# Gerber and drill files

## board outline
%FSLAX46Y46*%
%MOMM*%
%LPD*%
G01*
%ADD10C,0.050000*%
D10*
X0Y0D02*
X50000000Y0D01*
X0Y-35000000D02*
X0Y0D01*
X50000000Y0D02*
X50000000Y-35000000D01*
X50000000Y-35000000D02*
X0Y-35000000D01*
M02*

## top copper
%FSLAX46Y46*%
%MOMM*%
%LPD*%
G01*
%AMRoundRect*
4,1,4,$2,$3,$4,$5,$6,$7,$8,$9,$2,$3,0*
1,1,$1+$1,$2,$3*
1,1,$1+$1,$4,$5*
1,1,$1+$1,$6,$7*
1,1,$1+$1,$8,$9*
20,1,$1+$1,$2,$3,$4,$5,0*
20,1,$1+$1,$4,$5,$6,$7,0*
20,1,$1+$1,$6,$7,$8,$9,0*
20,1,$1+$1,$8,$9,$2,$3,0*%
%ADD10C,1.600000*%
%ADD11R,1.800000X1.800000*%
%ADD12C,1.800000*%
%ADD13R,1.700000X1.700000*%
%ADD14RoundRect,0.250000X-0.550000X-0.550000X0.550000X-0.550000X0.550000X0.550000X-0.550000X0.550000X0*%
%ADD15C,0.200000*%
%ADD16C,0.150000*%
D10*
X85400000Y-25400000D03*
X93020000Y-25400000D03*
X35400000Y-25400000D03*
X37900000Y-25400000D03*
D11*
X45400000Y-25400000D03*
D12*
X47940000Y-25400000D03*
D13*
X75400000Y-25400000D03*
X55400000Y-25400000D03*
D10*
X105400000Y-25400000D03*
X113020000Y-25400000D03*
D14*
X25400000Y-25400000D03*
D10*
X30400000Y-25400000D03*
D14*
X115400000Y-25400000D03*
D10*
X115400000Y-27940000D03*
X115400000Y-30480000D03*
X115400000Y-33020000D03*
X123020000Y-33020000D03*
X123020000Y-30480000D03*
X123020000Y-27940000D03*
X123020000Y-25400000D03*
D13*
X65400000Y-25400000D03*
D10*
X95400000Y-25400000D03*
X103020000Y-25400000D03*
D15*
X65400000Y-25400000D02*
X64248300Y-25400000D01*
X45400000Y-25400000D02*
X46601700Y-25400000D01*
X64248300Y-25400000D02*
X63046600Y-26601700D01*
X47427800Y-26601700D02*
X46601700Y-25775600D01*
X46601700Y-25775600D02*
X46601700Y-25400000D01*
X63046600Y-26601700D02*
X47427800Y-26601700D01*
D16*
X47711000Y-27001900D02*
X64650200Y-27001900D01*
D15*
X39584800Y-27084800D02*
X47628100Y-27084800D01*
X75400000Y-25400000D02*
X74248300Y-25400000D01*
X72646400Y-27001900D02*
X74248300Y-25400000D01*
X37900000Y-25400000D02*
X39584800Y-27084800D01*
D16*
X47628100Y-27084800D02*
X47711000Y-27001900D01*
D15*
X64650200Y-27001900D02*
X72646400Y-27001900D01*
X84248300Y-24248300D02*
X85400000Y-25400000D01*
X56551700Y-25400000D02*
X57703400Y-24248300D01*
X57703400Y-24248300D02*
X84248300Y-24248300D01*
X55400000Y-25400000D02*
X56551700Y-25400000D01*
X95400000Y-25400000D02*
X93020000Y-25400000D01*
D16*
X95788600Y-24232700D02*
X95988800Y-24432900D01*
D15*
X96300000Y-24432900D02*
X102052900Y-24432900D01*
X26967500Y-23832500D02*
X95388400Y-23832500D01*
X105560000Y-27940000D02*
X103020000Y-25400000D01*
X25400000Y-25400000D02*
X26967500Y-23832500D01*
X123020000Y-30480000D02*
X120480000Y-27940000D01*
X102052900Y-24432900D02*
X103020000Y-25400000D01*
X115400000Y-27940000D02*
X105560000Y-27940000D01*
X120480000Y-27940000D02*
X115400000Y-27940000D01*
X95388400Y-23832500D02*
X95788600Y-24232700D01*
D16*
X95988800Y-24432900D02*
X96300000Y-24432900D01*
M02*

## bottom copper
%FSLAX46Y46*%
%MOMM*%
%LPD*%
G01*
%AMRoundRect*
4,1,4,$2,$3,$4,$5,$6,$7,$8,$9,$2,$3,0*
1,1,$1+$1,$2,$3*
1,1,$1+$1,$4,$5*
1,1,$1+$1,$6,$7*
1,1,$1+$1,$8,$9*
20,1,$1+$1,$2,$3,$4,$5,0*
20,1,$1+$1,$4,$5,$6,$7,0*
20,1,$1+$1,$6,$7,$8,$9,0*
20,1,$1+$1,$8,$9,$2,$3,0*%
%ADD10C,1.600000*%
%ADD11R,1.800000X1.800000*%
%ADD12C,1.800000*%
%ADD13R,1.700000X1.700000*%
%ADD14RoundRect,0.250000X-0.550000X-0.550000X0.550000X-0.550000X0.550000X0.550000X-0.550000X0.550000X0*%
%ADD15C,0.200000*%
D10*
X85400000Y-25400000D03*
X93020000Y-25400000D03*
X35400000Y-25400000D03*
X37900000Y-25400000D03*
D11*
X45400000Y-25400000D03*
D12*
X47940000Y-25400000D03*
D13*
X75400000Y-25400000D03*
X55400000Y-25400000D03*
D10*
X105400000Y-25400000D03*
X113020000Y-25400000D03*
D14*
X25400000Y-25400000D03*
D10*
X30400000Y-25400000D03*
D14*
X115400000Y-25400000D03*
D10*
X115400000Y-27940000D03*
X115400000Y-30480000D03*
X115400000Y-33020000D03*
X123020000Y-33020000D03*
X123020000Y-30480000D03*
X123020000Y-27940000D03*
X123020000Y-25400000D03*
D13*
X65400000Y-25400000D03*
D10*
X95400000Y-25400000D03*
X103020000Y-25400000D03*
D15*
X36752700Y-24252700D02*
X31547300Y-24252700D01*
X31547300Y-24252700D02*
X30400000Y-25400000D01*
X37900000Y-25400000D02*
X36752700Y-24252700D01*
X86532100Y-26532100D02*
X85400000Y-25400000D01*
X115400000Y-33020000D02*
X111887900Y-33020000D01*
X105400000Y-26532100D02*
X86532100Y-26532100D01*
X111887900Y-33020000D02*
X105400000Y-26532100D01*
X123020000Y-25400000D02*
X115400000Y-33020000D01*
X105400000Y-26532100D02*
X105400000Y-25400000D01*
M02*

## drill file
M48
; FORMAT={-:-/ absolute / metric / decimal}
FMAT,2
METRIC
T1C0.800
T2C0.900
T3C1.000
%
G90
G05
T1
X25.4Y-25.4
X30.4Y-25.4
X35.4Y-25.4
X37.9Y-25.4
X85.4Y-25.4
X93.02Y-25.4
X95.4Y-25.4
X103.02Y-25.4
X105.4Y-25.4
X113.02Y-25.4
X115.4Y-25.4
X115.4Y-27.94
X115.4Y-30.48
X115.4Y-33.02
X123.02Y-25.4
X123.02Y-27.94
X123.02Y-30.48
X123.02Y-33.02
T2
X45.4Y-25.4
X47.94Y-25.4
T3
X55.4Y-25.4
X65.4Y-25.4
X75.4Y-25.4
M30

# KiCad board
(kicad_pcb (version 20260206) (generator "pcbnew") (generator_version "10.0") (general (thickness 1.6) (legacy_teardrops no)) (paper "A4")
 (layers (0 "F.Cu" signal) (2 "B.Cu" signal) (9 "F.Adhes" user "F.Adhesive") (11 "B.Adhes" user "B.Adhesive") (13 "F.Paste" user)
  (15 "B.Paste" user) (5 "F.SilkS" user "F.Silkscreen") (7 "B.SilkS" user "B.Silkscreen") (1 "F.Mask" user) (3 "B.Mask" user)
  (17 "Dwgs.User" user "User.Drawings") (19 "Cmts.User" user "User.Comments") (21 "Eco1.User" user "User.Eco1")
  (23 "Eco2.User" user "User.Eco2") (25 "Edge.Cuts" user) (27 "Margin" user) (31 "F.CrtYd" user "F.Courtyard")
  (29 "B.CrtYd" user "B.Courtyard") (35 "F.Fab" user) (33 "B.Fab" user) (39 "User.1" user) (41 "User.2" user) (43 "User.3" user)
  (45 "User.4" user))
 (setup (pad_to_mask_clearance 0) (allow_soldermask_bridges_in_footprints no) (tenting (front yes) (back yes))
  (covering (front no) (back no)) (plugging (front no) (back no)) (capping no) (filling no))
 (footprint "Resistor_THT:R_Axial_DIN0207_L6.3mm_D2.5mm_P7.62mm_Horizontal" (layer "F.Cu") (at 85.4 25.4)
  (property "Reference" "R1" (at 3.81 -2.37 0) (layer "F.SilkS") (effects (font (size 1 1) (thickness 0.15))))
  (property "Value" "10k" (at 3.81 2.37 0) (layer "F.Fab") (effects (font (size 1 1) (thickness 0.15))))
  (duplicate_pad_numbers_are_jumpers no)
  (pad "1" thru_hole circle (at 0 0) (size 1.6 1.6) (drill 0.8) (layers "*.Cu" "*.Mask") (remove_unused_layers no) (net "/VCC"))
  (pad "2" thru_hole circle (at 7.62 0) (size 1.6 1.6) (drill 0.8) (layers "*.Cu" "*.Mask") (remove_unused_layers no) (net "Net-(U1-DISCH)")))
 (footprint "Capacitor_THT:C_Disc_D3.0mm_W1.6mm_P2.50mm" (layer "F.Cu") (at 35.4 25.4)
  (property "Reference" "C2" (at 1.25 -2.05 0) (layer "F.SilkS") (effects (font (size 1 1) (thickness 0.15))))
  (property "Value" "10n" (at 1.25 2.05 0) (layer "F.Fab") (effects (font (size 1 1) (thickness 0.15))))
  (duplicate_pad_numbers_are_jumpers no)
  (pad "1" thru_hole circle (at 0 0) (size 1.6 1.6) (drill 0.8) (layers "*.Cu" "*.Mask") (remove_unused_layers no) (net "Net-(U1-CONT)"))
  (pad "2" thru_hole circle (at 2.5 0) (size 1.6 1.6) (drill 0.8) (layers "*.Cu" "*.Mask") (remove_unused_layers no) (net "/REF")))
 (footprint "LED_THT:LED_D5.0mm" (layer "F.Cu") (at 45.4 25.4)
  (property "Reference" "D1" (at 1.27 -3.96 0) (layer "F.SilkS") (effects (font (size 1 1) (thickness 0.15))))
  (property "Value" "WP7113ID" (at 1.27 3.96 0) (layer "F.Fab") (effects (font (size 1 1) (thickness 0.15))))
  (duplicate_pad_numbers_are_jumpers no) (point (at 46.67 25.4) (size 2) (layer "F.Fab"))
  (pad "1" thru_hole rect (at 0 0) (size 1.8 1.8) (drill 0.9) (layers "*.Cu" "*.Mask") (remove_unused_layers no) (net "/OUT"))
  (pad "2" thru_hole circle (at 2.54 0) (size 1.8 1.8) (drill 0.9) (layers "*.Cu" "*.Mask") (remove_unused_layers no) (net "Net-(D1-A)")))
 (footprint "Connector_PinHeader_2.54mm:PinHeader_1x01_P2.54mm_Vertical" (layer "F.Cu") (at 75.4 25.4)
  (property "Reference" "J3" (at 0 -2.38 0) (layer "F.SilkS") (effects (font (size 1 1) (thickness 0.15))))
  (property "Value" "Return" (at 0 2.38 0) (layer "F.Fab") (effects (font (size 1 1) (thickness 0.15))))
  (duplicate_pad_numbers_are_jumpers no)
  (pad "1" thru_hole rect (at 0 0) (size 1.7 1.7) (drill 1) (layers "*.Cu" "*.Mask") (remove_unused_layers no) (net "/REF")))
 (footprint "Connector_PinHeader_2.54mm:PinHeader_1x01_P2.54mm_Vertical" (layer "F.Cu") (at 55.4 25.4)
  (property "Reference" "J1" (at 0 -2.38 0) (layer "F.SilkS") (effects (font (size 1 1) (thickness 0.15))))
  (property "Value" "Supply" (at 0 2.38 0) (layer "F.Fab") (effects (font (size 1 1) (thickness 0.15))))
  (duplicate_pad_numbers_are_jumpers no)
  (pad "1" thru_hole rect (at 0 0) (size 1.7 1.7) (drill 1) (layers "*.Cu" "*.Mask") (remove_unused_layers no) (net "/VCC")))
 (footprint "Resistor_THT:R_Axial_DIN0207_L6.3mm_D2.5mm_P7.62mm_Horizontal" (layer "F.Cu") (at 105.4 25.4)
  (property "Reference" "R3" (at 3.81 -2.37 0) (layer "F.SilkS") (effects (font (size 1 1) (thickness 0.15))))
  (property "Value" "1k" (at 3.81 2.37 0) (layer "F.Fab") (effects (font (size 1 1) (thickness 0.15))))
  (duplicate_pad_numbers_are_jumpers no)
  (pad "1" thru_hole circle (at 0 0) (size 1.6 1.6) (drill 0.8) (layers "*.Cu" "*.Mask") (remove_unused_layers no) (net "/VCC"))
  (pad "2" thru_hole circle (at 7.62 0) (size 1.6 1.6) (drill 0.8) (layers "*.Cu" "*.Mask") (remove_unused_layers no) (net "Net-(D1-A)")))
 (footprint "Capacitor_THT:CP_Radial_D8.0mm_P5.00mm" (layer "F.Cu") (at 25.4 25.4)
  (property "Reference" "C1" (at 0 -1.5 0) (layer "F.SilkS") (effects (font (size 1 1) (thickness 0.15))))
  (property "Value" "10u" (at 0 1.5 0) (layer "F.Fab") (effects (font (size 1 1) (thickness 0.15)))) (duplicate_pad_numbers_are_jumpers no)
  (pad "1" thru_hole roundrect (at 0 0) (size 1.6 1.6) (drill 0.8) (layers "*.Cu" "*.Mask") (remove_unused_layers no)
   (roundrect_rratio 0.15625) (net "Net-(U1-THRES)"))
  (pad "2" thru_hole circle (at 5 0) (size 1.6 1.6) (drill 0.8) (layers "*.Cu" "*.Mask") (remove_unused_layers no) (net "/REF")))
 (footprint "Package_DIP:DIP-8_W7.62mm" (layer "F.Cu") (at 115.4 25.4)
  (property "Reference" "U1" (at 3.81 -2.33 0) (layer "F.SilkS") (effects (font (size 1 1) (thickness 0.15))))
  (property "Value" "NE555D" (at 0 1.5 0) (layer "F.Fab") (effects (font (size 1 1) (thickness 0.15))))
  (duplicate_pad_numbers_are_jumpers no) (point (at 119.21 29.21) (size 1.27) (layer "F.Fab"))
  (pad "1" thru_hole roundrect (at 0 0) (size 1.6 1.6) (drill 0.8) (layers "*.Cu" "*.Mask") (remove_unused_layers no)
   (roundrect_rratio 0.15625) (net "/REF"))
  (pad "2" thru_hole circle (at 0 2.54) (size 1.6 1.6) (drill 0.8) (layers "*.Cu" "*.Mask") (remove_unused_layers no) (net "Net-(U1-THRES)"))
  (pad "3" thru_hole circle (at 0 5.08) (size 1.6 1.6) (drill 0.8) (layers "*.Cu" "*.Mask") (remove_unused_layers no) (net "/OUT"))
  (pad "4" thru_hole circle (at 0 7.62) (size 1.6 1.6) (drill 0.8) (layers "*.Cu" "*.Mask") (remove_unused_layers no) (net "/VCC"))
  (pad "5" thru_hole circle (at 7.62 7.62) (size 1.6 1.6) (drill 0.8) (layers "*.Cu" "*.Mask") (remove_unused_layers no)
   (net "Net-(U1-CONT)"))
  (pad "6" thru_hole circle (at 7.62 5.08) (size 1.6 1.6) (drill 0.8) (layers "*.Cu" "*.Mask") (remove_unused_layers no)
   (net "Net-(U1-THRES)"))
  (pad "7" thru_hole circle (at 7.62 2.54) (size 1.6 1.6) (drill 0.8) (layers "*.Cu" "*.Mask") (remove_unused_layers no)
   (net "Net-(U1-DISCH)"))
  (pad "8" thru_hole circle (at 7.62 0) (size 1.6 1.6) (drill 0.8) (layers "*.Cu" "*.Mask") (remove_unused_layers no) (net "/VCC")))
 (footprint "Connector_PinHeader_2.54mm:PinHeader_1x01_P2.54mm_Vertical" (layer "F.Cu") (at 65.4 25.4)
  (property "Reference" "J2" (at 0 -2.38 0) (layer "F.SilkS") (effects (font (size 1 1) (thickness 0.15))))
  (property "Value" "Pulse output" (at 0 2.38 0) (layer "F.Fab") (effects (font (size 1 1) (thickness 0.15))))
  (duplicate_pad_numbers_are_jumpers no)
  (pad "1" thru_hole rect (at 0 0) (size 1.7 1.7) (drill 1) (layers "*.Cu" "*.Mask") (remove_unused_layers no) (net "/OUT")))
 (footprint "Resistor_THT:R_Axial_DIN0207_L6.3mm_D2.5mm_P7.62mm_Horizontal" (layer "F.Cu") (at 95.4 25.4)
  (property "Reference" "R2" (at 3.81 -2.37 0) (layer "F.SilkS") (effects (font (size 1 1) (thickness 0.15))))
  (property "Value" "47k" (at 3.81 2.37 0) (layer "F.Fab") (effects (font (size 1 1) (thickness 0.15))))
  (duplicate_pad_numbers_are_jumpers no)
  (pad "1" thru_hole circle (at 0 0) (size 1.6 1.6) (drill 0.8) (layers "*.Cu" "*.Mask") (remove_unused_layers no) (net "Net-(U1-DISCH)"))
  (pad "2" thru_hole circle (at 7.62 0) (size 1.6 1.6) (drill 0.8) (layers "*.Cu" "*.Mask") (remove_unused_layers no) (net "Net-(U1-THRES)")))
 (gr_line (start 0 0) (end 50 0) (stroke (width 0.05) (type default)) (layer "Edge.Cuts"))
 (gr_line (start 0 35) (end 0 0) (stroke (width 0.05) (type default)) (layer "Edge.Cuts"))
 (gr_line (start 50 0) (end 50 35) (stroke (width 0.05) (type default)) (layer "Edge.Cuts"))
 (gr_line (start 50 35) (end 0 35) (stroke (width 0.05) (type default)) (layer "Edge.Cuts"))
 (segment (start 65.4 25.4) (end 64.2483 25.4) (width 0.2) (layer "F.Cu") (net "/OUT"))
 (segment (start 45.4 25.4) (end 46.6017 25.4) (width 0.2) (layer "F.Cu") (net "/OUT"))
 (segment (start 64.2483 25.4) (end 63.0466 26.6017) (width 0.2) (layer "F.Cu") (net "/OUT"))
 (segment (start 47.4278 26.6017) (end 46.6017 25.7756) (width 0.2) (layer "F.Cu") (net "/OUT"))
 (segment (start 46.6017 25.7756) (end 46.6017 25.4) (width 0.2) (layer "F.Cu") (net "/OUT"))
 (segment (start 63.0466 26.6017) (end 47.4278 26.6017) (width 0.2) (layer "F.Cu") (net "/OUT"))
 (segment (start 47.711 27.0019) (end 64.6502 27.0019) (width 0.15) (layer "F.Cu") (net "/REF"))
 (segment (start 39.5848 27.0848) (end 47.6281 27.0848) (width 0.2) (layer "F.Cu") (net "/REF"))
 (segment (start 75.4 25.4) (end 74.2483 25.4) (width 0.2) (layer "F.Cu") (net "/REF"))
 (segment (start 72.6464 27.0019) (end 74.2483 25.4) (width 0.2) (layer "F.Cu") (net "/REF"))
 (segment (start 37.9 25.4) (end 39.5848 27.0848) (width 0.2) (layer "F.Cu") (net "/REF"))
 (segment (start 47.6281 27.0848) (end 47.711 27.0019) (width 0.15) (layer "F.Cu") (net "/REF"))
 (segment (start 64.6502 27.0019) (end 72.6464 27.0019) (width 0.2) (layer "F.Cu") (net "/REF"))
 (segment (start 36.7527 24.2527) (end 31.5473 24.2527) (width 0.2) (layer "B.Cu") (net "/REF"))
 (segment (start 31.5473 24.2527) (end 30.4 25.4) (width 0.2) (layer "B.Cu") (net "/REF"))
 (segment (start 37.9 25.4) (end 36.7527 24.2527) (width 0.2) (layer "B.Cu") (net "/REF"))
 (segment (start 84.2483 24.2483) (end 85.4 25.4) (width 0.2) (layer "F.Cu") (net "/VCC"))
 (segment (start 56.5517 25.4) (end 57.7034 24.2483) (width 0.2) (layer "F.Cu") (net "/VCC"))
 (segment (start 57.7034 24.2483) (end 84.2483 24.2483) (width 0.2) (layer "F.Cu") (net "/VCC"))
 (segment (start 55.4 25.4) (end 56.5517 25.4) (width 0.2) (layer "F.Cu") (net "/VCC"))
 (segment (start 86.5321 26.5321) (end 85.4 25.4) (width 0.2) (layer "B.Cu") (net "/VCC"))
 (segment (start 115.4 33.02) (end 111.8879 33.02) (width 0.2) (layer "B.Cu") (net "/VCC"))
 (segment (start 105.4 26.5321) (end 86.5321 26.5321) (width 0.2) (layer "B.Cu") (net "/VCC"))
 (segment (start 111.8879 33.02) (end 105.4 26.5321) (width 0.2) (layer "B.Cu") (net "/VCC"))
 (segment (start 123.02 25.4) (end 115.4 33.02) (width 0.2) (layer "B.Cu") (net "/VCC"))
 (segment (start 105.4 26.5321) (end 105.4 25.4) (width 0.2) (layer "B.Cu") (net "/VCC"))
 (segment (start 95.4 25.4) (end 93.02 25.4) (width 0.2) (layer "F.Cu") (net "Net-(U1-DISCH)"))
 (segment (start 95.7886 24.2327) (end 95.9888 24.4329) (width 0.15) (layer "F.Cu") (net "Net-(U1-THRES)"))
 (segment (start 96.3 24.4329) (end 102.0529 24.4329) (width 0.2) (layer "F.Cu") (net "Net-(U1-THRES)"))
 (segment (start 26.9675 23.8325) (end 95.3884 23.8325) (width 0.2) (layer "F.Cu") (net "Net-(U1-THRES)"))
 (segment (start 105.56 27.94) (end 103.02 25.4) (width 0.2) (layer "F.Cu") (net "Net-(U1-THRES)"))
 (segment (start 25.4 25.4) (end 26.9675 23.8325) (width 0.2) (layer "F.Cu") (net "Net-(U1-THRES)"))
 (segment (start 123.02 30.48) (end 120.48 27.94) (width 0.2) (layer "F.Cu") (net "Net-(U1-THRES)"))
 (segment (start 102.0529 24.4329) (end 103.02 25.4) (width 0.2) (layer "F.Cu") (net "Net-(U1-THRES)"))
 (segment (start 115.4 27.94) (end 105.56 27.94) (width 0.2) (layer "F.Cu") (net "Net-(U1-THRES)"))
 (segment (start 120.48 27.94) (end 115.4 27.94) (width 0.2) (layer "F.Cu") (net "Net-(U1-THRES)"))
 (segment (start 95.3884 23.8325) (end 95.7886 24.2327) (width 0.2) (layer "F.Cu") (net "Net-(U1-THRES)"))
 (segment (start 95.9888 24.4329) (end 96.3 24.4329) (width 0.15) (layer "F.Cu") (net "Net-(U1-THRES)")))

